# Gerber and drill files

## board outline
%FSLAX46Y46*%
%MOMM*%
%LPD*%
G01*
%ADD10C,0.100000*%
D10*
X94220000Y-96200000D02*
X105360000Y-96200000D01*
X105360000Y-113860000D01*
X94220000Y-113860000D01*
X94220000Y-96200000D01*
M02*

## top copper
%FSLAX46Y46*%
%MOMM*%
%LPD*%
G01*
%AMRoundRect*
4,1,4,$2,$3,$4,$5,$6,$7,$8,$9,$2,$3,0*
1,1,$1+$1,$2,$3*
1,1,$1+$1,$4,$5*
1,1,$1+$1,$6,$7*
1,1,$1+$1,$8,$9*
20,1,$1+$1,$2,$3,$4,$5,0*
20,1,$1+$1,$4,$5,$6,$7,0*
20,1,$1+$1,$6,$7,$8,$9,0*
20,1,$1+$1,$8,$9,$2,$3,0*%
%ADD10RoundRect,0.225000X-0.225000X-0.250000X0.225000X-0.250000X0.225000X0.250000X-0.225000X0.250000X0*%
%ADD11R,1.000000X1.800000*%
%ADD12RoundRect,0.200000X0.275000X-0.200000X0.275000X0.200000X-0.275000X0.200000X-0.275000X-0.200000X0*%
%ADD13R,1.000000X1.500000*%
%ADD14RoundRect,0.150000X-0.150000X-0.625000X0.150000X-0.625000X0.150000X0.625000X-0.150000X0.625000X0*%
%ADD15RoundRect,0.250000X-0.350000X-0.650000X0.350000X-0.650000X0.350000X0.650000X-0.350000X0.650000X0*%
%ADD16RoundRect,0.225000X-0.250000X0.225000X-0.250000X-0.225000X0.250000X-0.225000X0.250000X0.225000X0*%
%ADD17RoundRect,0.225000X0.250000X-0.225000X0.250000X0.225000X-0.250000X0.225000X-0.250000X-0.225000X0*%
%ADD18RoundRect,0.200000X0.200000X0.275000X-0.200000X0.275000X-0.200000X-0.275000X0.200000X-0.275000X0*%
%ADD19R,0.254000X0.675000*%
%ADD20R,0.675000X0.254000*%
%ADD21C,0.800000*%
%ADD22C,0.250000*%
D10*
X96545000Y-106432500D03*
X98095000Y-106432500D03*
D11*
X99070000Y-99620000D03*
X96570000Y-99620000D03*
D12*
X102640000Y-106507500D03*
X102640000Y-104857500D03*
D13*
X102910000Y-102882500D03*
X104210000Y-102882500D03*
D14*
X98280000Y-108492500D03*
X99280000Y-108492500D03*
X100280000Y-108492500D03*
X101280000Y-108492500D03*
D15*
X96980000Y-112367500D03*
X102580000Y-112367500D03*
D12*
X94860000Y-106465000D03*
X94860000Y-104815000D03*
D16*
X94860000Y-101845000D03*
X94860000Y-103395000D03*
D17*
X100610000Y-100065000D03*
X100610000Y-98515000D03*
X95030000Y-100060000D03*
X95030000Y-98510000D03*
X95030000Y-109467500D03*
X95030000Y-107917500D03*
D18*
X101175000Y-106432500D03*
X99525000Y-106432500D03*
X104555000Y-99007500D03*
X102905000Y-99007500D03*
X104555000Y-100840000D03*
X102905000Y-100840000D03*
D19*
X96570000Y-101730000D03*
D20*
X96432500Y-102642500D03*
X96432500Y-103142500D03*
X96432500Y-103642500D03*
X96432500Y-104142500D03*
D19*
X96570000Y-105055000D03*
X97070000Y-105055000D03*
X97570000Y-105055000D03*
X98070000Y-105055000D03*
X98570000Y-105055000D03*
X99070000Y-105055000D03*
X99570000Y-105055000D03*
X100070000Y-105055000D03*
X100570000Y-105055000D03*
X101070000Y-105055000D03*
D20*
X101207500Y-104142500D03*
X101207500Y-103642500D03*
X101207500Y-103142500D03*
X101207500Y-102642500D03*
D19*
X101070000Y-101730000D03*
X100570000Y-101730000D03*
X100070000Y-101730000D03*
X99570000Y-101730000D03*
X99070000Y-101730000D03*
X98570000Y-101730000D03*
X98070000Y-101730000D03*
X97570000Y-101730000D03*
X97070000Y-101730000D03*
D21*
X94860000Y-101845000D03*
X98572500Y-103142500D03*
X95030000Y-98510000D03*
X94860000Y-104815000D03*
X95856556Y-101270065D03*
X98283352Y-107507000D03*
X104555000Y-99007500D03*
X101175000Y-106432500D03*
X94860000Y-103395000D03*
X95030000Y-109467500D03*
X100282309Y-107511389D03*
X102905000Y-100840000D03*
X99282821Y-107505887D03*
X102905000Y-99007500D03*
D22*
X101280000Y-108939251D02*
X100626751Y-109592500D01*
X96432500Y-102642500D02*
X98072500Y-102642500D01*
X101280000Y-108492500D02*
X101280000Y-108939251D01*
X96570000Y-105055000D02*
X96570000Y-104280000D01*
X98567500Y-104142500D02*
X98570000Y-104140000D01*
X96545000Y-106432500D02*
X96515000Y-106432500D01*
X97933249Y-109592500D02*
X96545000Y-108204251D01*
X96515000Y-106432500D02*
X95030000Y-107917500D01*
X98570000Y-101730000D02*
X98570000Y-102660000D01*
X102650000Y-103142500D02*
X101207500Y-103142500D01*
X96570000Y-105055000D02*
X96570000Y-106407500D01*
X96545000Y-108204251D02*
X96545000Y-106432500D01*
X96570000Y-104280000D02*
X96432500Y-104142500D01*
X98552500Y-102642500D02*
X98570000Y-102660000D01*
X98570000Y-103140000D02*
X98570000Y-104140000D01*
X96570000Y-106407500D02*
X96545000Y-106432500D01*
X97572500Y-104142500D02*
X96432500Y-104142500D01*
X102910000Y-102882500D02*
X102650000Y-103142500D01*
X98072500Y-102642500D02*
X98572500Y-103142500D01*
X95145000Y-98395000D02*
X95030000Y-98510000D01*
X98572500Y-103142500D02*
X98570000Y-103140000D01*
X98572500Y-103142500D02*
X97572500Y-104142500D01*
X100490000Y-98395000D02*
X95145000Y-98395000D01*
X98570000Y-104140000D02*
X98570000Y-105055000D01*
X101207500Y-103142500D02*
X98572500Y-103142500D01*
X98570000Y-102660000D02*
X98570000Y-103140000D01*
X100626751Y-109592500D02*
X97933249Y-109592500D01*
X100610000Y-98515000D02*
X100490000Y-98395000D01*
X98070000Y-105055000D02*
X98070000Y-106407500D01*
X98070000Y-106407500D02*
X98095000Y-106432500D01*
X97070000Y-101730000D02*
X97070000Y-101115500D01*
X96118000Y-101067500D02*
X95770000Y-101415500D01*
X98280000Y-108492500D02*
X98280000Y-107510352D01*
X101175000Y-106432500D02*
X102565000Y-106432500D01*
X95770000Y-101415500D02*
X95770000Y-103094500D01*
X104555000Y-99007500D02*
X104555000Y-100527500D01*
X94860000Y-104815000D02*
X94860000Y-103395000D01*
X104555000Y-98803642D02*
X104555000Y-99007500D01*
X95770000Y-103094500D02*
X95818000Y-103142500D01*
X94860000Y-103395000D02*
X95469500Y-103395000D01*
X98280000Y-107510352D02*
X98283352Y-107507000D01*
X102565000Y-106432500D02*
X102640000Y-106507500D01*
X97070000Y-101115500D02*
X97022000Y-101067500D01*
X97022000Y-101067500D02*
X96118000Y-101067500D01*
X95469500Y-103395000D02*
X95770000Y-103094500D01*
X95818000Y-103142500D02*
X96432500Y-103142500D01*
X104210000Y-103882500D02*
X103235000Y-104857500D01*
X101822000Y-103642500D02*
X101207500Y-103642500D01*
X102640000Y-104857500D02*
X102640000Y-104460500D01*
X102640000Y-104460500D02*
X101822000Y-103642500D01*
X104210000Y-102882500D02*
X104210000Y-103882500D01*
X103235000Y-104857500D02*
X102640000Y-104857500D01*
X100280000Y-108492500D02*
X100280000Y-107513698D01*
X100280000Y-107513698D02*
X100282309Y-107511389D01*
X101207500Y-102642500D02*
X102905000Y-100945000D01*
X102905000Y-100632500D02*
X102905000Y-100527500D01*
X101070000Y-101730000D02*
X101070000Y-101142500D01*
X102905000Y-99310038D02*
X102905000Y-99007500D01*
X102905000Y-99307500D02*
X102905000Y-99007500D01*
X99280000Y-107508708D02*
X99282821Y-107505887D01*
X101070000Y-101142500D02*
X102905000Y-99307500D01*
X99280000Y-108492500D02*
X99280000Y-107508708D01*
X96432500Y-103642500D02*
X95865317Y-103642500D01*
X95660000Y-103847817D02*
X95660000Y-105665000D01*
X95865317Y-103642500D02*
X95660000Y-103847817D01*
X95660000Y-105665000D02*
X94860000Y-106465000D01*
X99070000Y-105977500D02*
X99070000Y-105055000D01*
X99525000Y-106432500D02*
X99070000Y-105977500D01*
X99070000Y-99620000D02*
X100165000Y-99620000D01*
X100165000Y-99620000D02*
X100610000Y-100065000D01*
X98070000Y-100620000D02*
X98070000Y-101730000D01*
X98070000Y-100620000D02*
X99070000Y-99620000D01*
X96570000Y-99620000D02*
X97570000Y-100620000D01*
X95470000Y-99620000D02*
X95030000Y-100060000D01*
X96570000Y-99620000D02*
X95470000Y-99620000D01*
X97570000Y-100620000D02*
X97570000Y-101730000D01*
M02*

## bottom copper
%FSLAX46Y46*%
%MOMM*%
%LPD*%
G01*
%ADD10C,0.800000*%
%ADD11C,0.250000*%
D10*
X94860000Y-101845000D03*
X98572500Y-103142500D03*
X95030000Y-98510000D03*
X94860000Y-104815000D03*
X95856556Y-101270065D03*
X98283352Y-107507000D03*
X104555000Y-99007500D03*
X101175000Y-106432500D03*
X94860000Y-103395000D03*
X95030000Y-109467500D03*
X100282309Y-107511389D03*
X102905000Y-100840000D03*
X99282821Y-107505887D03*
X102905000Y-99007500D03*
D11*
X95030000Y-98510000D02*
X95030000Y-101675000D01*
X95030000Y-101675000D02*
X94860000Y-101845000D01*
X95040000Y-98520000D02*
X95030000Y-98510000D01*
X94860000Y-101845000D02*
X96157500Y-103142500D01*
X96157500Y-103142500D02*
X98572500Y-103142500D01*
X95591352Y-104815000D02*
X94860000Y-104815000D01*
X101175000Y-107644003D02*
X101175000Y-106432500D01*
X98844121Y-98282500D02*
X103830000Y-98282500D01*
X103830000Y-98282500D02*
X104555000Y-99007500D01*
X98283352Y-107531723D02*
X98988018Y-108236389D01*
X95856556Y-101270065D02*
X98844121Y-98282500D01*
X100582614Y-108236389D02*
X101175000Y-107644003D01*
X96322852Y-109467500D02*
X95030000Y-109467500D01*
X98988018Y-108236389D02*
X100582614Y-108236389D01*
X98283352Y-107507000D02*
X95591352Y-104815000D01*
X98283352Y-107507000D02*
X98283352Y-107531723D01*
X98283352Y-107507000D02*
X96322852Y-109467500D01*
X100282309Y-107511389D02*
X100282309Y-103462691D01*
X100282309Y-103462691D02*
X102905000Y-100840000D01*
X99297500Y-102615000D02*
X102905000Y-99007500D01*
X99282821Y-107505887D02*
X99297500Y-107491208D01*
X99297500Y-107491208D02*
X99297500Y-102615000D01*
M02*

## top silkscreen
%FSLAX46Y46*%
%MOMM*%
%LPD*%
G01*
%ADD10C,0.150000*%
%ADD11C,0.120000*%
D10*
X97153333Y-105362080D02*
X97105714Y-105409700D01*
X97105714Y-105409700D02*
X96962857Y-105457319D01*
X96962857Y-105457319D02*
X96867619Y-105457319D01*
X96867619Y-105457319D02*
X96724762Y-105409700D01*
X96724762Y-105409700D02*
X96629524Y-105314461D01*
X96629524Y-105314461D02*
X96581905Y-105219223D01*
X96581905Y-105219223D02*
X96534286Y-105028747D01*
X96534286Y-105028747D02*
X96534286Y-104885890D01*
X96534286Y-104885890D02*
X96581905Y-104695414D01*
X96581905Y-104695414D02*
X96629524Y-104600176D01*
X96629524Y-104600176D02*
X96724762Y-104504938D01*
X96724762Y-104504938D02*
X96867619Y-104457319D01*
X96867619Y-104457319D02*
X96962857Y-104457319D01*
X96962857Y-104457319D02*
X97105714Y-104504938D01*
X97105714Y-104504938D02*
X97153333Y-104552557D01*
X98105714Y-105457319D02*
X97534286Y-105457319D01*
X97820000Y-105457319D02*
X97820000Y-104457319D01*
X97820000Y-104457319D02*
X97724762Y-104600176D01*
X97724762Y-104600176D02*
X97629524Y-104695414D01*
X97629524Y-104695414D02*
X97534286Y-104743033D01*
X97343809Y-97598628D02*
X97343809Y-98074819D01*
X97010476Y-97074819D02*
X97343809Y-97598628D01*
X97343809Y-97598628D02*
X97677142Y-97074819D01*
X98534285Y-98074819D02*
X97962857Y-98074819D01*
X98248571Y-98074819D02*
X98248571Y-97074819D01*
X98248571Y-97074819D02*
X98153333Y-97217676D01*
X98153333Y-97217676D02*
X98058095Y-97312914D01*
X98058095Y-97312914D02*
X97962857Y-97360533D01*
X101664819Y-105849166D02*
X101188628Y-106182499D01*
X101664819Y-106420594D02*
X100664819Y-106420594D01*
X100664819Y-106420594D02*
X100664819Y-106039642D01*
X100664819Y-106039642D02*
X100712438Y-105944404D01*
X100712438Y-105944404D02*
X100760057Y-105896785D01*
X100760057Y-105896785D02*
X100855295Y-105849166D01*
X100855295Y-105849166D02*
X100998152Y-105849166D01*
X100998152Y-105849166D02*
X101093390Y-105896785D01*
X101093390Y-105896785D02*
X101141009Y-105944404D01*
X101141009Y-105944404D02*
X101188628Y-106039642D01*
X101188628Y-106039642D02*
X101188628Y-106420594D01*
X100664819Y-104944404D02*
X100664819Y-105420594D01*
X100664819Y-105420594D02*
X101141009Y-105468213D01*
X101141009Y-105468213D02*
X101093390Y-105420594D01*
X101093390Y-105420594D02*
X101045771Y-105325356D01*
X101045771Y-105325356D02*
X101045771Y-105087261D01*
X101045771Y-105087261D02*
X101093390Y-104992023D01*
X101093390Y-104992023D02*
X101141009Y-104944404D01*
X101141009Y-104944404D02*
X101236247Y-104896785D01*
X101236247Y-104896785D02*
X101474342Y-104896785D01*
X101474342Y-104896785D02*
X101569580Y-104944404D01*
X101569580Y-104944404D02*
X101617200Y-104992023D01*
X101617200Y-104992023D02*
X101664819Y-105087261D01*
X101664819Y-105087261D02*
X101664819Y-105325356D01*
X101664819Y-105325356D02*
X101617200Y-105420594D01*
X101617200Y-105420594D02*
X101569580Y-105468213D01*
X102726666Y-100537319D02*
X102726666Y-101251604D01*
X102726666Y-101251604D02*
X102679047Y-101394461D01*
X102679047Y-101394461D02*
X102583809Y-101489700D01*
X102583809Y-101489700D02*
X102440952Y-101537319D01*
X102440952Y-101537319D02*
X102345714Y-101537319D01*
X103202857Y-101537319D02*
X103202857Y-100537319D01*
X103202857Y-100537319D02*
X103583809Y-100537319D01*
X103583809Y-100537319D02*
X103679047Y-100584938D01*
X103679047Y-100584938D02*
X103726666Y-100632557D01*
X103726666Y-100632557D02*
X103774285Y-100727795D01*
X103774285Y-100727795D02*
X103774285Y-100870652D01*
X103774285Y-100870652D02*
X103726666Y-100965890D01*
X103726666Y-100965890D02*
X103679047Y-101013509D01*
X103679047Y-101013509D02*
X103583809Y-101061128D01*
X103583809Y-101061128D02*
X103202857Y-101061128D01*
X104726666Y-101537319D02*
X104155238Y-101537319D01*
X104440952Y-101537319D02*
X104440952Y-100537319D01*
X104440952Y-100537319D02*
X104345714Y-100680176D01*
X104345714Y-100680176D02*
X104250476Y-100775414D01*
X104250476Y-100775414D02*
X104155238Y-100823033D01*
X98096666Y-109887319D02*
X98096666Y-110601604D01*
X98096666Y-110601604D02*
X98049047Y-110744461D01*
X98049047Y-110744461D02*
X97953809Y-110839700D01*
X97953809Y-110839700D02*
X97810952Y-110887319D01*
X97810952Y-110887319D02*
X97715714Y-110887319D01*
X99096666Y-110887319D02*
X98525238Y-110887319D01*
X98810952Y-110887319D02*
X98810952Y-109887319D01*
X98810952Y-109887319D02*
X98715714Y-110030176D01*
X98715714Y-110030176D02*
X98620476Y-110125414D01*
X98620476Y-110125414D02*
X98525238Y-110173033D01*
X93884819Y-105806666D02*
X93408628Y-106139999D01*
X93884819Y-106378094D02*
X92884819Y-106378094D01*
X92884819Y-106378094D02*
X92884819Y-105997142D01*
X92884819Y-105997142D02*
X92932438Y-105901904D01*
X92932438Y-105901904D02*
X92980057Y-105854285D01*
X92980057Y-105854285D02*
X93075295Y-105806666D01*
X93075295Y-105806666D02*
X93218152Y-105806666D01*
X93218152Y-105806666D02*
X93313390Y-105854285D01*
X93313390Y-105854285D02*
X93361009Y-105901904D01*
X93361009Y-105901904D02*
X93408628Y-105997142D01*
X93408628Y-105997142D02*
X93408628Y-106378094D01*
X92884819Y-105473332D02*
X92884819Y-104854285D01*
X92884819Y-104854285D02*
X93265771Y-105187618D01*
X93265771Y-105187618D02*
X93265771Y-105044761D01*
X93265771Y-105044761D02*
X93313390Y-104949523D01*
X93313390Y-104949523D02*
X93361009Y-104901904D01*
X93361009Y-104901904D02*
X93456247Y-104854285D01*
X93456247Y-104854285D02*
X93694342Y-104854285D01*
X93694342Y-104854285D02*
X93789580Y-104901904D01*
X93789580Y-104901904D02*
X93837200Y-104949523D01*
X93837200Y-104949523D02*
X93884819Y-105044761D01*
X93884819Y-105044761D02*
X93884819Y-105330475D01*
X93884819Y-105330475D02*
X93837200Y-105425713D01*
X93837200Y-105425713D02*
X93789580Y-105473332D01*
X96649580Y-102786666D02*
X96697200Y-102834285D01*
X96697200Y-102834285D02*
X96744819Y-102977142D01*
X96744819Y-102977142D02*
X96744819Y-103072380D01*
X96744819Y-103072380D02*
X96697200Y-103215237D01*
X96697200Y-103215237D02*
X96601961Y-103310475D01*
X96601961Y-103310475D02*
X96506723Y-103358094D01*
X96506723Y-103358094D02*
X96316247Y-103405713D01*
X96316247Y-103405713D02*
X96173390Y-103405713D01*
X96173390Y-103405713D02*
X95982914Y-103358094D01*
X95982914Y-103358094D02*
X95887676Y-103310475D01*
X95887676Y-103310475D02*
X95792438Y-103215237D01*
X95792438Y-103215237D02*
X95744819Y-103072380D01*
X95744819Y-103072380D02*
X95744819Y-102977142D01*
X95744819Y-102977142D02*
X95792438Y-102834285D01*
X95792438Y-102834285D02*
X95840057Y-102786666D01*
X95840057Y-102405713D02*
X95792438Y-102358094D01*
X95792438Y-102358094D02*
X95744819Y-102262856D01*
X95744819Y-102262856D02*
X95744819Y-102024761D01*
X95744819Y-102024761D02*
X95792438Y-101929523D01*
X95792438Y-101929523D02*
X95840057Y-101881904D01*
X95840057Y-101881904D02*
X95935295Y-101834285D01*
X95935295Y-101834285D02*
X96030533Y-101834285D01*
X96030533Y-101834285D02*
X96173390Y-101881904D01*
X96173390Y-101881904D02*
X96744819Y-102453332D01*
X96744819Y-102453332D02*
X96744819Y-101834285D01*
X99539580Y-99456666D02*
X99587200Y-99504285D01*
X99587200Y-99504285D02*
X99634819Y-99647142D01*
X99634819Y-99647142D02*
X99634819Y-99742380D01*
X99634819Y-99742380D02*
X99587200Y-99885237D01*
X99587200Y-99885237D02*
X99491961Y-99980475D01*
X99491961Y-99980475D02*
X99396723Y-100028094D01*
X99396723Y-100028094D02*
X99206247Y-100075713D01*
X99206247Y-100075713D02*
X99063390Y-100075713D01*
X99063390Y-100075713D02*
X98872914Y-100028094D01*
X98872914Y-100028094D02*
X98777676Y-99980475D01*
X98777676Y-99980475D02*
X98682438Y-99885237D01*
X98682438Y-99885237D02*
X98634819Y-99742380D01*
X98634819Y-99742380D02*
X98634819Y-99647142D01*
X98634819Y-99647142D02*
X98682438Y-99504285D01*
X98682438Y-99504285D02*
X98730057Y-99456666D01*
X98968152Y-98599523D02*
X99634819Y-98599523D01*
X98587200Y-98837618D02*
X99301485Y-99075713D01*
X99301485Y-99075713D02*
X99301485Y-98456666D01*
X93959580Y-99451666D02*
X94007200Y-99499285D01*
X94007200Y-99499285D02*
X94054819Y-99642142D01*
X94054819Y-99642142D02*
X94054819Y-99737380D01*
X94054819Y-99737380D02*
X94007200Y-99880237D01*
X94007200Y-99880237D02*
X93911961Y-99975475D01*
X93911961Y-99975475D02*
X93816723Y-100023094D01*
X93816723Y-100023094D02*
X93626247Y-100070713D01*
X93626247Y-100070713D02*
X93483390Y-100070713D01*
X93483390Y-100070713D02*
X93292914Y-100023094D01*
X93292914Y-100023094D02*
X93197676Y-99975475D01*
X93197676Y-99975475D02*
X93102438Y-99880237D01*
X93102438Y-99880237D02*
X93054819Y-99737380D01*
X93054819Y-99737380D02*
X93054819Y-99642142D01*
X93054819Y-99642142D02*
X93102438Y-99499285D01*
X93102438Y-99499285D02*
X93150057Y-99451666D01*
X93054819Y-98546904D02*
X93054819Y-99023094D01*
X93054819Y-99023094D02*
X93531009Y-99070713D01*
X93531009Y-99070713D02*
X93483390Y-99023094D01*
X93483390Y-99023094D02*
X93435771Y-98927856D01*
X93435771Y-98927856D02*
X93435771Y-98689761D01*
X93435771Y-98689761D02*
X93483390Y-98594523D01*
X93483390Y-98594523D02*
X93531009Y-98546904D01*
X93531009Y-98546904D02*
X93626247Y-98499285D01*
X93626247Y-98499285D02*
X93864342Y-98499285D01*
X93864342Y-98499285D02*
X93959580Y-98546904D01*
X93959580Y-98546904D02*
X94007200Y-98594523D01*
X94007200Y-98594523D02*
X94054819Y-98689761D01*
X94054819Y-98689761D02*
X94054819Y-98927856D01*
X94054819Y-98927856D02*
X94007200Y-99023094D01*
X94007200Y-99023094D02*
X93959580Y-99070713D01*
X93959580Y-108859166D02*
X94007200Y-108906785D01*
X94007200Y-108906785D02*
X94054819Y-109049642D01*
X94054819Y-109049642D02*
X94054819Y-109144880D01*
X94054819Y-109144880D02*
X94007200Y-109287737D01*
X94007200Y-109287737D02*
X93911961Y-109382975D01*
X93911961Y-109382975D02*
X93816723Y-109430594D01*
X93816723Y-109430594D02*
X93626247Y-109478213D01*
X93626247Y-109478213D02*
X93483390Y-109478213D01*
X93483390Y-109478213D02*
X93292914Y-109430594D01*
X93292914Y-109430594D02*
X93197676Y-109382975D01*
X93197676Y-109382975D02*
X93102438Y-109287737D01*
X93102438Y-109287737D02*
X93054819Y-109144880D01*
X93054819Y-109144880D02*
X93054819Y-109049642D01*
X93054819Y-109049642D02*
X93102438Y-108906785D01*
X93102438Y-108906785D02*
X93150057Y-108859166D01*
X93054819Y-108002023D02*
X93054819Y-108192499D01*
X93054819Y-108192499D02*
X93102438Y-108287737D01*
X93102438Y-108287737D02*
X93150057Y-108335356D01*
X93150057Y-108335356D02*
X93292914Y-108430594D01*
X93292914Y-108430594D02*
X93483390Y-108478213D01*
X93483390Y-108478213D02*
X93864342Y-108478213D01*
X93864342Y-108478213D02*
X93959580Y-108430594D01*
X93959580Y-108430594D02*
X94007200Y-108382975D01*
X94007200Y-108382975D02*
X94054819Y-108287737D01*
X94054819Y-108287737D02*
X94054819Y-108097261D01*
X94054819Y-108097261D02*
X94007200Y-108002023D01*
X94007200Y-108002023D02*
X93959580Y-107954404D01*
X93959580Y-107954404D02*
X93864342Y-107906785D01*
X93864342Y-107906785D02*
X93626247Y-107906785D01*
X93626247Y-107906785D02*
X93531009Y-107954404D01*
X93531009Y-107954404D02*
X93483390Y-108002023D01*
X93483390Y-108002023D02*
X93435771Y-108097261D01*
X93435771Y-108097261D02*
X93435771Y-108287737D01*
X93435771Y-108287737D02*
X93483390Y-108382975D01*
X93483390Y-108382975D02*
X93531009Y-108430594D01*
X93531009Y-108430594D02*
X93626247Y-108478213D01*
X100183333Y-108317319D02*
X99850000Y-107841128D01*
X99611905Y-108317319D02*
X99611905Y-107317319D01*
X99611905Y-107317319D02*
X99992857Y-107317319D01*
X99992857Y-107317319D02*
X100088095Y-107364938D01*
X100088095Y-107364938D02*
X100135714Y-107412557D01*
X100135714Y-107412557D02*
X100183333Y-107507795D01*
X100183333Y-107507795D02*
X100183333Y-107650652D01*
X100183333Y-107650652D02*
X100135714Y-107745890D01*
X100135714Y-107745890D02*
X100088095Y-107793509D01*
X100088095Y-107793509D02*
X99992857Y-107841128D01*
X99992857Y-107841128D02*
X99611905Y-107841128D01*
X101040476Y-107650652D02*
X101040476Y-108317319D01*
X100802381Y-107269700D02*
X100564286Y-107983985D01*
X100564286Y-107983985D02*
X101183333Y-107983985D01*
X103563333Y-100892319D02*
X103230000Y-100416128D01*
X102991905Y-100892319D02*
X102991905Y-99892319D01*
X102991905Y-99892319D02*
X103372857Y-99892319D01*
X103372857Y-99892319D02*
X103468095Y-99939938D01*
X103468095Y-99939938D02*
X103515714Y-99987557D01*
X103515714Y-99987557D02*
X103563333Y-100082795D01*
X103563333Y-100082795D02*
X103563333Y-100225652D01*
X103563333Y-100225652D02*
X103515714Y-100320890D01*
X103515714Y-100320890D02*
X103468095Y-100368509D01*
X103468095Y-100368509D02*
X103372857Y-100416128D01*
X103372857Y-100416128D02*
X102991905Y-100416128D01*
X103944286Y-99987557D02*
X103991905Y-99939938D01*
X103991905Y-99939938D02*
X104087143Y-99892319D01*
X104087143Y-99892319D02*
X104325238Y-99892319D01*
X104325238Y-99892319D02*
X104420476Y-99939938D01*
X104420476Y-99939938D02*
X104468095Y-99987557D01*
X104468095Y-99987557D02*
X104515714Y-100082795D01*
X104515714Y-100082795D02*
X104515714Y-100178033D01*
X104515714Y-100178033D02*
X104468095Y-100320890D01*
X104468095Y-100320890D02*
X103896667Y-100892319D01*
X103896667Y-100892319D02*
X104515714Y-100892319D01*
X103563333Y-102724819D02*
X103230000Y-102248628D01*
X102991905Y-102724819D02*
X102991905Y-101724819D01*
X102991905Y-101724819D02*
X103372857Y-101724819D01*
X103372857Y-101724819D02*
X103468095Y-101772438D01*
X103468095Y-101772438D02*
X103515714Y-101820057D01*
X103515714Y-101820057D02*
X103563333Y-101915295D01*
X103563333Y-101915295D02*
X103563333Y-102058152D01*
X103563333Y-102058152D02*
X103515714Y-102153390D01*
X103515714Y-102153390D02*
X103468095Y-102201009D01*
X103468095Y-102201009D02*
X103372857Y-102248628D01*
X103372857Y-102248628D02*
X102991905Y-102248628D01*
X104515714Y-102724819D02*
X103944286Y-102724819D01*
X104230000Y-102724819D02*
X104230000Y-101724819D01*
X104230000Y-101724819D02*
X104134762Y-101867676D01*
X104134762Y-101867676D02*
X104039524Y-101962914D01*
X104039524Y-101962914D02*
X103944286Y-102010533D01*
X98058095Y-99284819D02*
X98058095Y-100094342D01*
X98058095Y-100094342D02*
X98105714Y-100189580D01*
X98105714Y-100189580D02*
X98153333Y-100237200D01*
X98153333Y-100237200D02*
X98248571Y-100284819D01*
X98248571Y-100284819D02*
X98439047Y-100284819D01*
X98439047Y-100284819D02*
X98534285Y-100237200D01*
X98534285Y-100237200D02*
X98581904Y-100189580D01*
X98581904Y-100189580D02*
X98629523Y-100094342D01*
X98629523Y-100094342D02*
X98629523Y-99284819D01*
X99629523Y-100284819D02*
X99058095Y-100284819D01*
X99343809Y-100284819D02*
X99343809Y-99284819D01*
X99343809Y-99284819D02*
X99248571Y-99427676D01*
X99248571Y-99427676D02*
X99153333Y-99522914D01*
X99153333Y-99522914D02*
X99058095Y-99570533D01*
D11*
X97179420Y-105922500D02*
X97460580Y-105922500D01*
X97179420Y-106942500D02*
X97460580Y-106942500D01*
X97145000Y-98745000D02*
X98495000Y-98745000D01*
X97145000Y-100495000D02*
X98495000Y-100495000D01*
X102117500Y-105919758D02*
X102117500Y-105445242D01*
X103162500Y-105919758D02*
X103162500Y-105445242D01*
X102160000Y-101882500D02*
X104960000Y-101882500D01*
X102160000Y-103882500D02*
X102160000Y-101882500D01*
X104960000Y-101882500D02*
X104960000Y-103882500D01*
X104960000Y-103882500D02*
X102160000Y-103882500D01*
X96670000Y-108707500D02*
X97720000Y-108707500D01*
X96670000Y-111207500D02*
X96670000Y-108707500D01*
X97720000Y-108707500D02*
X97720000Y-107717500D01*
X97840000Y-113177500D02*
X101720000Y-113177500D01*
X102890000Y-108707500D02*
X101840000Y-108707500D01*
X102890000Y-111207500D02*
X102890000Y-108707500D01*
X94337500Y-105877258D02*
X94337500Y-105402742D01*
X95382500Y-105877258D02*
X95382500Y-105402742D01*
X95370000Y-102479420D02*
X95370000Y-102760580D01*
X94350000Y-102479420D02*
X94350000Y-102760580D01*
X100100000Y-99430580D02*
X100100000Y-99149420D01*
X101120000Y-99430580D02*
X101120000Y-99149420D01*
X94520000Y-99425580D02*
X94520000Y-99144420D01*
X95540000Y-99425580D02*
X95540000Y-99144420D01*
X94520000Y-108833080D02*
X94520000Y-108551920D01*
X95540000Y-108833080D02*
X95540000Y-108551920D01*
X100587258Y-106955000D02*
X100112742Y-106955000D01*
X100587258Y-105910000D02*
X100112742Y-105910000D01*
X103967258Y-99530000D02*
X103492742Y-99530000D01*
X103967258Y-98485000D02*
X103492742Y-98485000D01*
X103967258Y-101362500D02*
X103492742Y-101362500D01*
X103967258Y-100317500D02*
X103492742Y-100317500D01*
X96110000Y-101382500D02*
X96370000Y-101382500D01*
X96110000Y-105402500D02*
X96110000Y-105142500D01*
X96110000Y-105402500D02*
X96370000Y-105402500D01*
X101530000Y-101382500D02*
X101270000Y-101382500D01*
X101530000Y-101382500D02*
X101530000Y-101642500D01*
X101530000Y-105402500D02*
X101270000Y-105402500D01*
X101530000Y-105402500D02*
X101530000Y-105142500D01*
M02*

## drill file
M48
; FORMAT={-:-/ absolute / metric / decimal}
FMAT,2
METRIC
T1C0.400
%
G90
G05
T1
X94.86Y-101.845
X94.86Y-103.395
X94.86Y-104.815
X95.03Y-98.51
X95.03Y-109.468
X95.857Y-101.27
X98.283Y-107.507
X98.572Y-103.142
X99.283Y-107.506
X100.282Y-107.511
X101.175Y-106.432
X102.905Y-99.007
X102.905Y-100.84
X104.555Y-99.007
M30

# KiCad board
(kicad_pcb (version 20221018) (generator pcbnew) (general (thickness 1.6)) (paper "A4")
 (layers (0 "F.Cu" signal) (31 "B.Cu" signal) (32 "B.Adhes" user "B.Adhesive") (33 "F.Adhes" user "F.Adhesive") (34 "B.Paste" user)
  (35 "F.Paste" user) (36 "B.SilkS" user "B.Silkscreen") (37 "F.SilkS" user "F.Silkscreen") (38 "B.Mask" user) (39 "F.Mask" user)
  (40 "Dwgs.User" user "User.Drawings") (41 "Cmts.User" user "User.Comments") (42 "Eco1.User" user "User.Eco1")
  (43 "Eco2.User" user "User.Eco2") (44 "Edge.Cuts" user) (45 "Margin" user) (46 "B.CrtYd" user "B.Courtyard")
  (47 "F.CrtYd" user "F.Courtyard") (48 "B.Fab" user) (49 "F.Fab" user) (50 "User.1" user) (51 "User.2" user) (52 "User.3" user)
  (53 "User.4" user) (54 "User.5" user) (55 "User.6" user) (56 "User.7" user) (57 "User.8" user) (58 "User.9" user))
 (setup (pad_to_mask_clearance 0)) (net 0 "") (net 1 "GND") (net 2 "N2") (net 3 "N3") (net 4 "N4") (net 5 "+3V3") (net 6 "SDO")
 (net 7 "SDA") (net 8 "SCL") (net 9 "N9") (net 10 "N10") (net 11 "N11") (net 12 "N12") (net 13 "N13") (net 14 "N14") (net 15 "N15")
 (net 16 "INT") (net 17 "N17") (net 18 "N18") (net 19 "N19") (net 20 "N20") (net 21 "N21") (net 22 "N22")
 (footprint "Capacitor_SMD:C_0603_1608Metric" (layer "F.Cu") (at 97.32 106.4325)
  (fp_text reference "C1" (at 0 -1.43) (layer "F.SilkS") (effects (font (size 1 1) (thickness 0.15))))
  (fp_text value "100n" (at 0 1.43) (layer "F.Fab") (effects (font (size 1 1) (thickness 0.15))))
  (fp_line (start -0.14058 -0.51) (end 0.14058 -0.51) (stroke (width 0.12) (type solid)) (layer "F.SilkS"))
  (fp_line (start -0.14058 0.51) (end 0.14058 0.51) (stroke (width 0.12) (type solid)) (layer "F.SilkS"))
  (pad "1" smd roundrect (at -0.775 0) (size 0.9 0.95) (layers "F.Cu" "F.Paste" "F.Mask") (roundrect_rratio 0.25) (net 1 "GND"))
  (pad "2" smd roundrect (at 0.775 0) (size 0.9 0.95) (layers "F.Cu" "F.Paste" "F.Mask") (roundrect_rratio 0.25) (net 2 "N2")))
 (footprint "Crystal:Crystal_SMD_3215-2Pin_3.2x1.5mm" (layer "F.Cu") (at 97.82 99.62)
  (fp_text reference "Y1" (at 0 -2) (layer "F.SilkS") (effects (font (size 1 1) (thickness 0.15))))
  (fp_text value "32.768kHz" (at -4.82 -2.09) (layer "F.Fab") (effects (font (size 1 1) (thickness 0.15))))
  (fp_line (start -0.675 -0.875) (end 0.675 -0.875) (stroke (width 0.12) (type solid)) (layer "F.SilkS"))
  (fp_line (start -0.675 0.875) (end 0.675 0.875) (stroke (width 0.12) (type solid)) (layer "F.SilkS"))
  (pad "1" smd rect (at 1.25 0) (size 1 1.8) (layers "F.Cu" "F.Paste" "F.Mask") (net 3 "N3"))
  (pad "2" smd rect (at -1.25 0) (size 1 1.8) (layers "F.Cu" "F.Paste" "F.Mask") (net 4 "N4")))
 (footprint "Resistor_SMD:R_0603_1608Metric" (layer "F.Cu") (at 102.64 105.6825 90)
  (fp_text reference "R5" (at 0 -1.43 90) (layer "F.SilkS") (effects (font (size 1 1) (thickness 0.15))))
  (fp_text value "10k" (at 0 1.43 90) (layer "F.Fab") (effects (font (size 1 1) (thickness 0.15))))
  (fp_line (start -0.237258 -0.5225) (end 0.237258 -0.5225) (stroke (width 0.12) (type solid)) (layer "F.SilkS"))
  (fp_line (start -0.237258 0.5225) (end 0.237258 0.5225) (stroke (width 0.12) (type solid)) (layer "F.SilkS"))
  (pad "1" smd roundrect (at -0.825 0 90) (size 0.8 0.95) (layers "F.Cu" "F.Paste" "F.Mask") (roundrect_rratio 0.25) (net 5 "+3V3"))
  (pad "2" smd roundrect (at 0.825 0 90) (size 0.8 0.95) (layers "F.Cu" "F.Paste" "F.Mask") (roundrect_rratio 0.25) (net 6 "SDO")))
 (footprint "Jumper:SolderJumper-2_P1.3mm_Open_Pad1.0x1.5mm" (layer "F.Cu") (at 103.56 102.8825)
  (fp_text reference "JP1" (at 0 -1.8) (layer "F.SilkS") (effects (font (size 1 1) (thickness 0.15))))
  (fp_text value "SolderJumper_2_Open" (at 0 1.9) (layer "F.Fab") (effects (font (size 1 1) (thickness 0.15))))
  (fp_line (start -1.4 -1) (end 1.4 -1) (stroke (width 0.12) (type solid)) (layer "F.SilkS"))
  (fp_line (start -1.4 1) (end -1.4 -1) (stroke (width 0.12) (type solid)) (layer "F.SilkS"))
  (fp_line (start 1.4 -1) (end 1.4 1) (stroke (width 0.12) (type solid)) (layer "F.SilkS"))
  (fp_line (start 1.4 1) (end -1.4 1) (stroke (width 0.12) (type solid)) (layer "F.SilkS"))
  (pad "1" smd rect (at -0.65 0) (size 1 1.5) (layers "F.Cu" "F.Mask") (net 1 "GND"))
  (pad "2" smd rect (at 0.65 0) (size 1 1.5) (layers "F.Cu" "F.Mask") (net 6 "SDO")))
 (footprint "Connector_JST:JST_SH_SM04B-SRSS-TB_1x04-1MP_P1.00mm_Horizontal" (layer "F.Cu") (at 99.78 110.4925)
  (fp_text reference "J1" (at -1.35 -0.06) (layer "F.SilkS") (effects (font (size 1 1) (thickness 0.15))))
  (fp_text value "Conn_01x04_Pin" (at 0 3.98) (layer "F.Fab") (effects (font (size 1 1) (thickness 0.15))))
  (fp_line (start -3.11 -1.785) (end -2.06 -1.785) (stroke (width 0.12) (type solid)) (layer "F.SilkS"))
  (fp_line (start -3.11 0.715) (end -3.11 -1.785) (stroke (width 0.12) (type solid)) (layer "F.SilkS"))
  (fp_line (start -2.06 -1.785) (end -2.06 -2.775) (stroke (width 0.12) (type solid)) (layer "F.SilkS"))
  (fp_line (start -1.94 2.685) (end 1.94 2.685) (stroke (width 0.12) (type solid)) (layer "F.SilkS"))
  (fp_line (start 3.11 -1.785) (end 2.06 -1.785) (stroke (width 0.12) (type solid)) (layer "F.SilkS"))
  (fp_line (start 3.11 0.715) (end 3.11 -1.785) (stroke (width 0.12) (type solid)) (layer "F.SilkS"))
  (pad "1" smd roundrect (at -1.5 -2) (size 0.6 1.55) (layers "F.Cu" "F.Paste" "F.Mask") (roundrect_rratio 0.25) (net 5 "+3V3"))
  (pad "2" smd roundrect (at -0.5 -2) (size 0.6 1.55) (layers "F.Cu" "F.Paste" "F.Mask") (roundrect_rratio 0.25) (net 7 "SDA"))
  (pad "3" smd roundrect (at 0.5 -2) (size 0.6 1.55) (layers "F.Cu" "F.Paste" "F.Mask") (roundrect_rratio 0.25) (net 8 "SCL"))
  (pad "4" smd roundrect (at 1.5 -2) (size 0.6 1.55) (layers "F.Cu" "F.Paste" "F.Mask") (roundrect_rratio 0.25) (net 1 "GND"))
  (pad "MP" smd roundrect (at -2.8 1.875) (size 1.2 1.8) (layers "F.Cu" "F.Paste" "F.Mask") (roundrect_rratio 0.208333))
  (pad "MP" smd roundrect (at 2.8 1.875) (size 1.2 1.8) (layers "F.Cu" "F.Paste" "F.Mask") (roundrect_rratio 0.208333)))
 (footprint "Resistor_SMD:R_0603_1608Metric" (layer "F.Cu") (at 94.86 105.64 90)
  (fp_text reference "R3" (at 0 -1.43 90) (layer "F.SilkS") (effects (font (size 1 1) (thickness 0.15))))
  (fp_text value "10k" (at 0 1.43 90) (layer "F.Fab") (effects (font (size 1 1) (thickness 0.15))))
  (fp_line (start -0.237258 -0.5225) (end 0.237258 -0.5225) (stroke (width 0.12) (type solid)) (layer "F.SilkS"))
  (fp_line (start -0.237258 0.5225) (end 0.237258 0.5225) (stroke (width 0.12) (type solid)) (layer "F.SilkS"))
  (pad "1" smd roundrect (at -0.825 0 90) (size 0.8 0.95) (layers "F.Cu" "F.Paste" "F.Mask") (roundrect_rratio 0.25) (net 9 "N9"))
  (pad "2" smd roundrect (at 0.825 0 90) (size 0.8 0.95) (layers "F.Cu" "F.Paste" "F.Mask") (roundrect_rratio 0.25) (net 5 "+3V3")))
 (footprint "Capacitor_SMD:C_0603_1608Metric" (layer "F.Cu") (at 94.86 102.62 -90)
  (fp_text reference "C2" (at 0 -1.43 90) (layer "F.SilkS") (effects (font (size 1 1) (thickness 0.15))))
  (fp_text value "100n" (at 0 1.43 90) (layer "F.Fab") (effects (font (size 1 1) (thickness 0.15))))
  (fp_line (start -0.14058 -0.51) (end 0.14058 -0.51) (stroke (width 0.12) (type solid)) (layer "F.SilkS"))
  (fp_line (start -0.14058 0.51) (end 0.14058 0.51) (stroke (width 0.12) (type solid)) (layer "F.SilkS"))
  (pad "1" smd roundrect (at -0.775 0 270) (size 0.9 0.95) (layers "F.Cu" "F.Paste" "F.Mask") (roundrect_rratio 0.25) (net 1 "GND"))
  (pad "2" smd roundrect (at 0.775 0 270) (size 0.9 0.95) (layers "F.Cu" "F.Paste" "F.Mask") (roundrect_rratio 0.25) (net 5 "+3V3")))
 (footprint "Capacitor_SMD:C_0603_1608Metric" (layer "F.Cu") (at 100.61 99.29 90)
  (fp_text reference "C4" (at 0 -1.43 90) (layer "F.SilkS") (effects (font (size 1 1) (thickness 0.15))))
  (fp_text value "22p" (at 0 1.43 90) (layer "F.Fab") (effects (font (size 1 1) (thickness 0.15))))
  (fp_line (start -0.14058 -0.51) (end 0.14058 -0.51) (stroke (width 0.12) (type solid)) (layer "F.SilkS"))
  (fp_line (start -0.14058 0.51) (end 0.14058 0.51) (stroke (width 0.12) (type solid)) (layer "F.SilkS"))
  (pad "1" smd roundrect (at -0.775 0 90) (size 0.9 0.95) (layers "F.Cu" "F.Paste" "F.Mask") (roundrect_rratio 0.25) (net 3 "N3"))
  (pad "2" smd roundrect (at 0.775 0 90) (size 0.9 0.95) (layers "F.Cu" "F.Paste" "F.Mask") (roundrect_rratio 0.25) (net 1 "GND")))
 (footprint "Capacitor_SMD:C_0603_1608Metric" (layer "F.Cu") (at 95.03 99.285 90)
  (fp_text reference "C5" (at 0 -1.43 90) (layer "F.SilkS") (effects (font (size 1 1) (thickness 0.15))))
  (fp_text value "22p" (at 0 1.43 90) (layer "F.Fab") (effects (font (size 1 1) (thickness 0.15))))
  (fp_line (start -0.14058 -0.51) (end 0.14058 -0.51) (stroke (width 0.12) (type solid)) (layer "F.SilkS"))
  (fp_line (start -0.14058 0.51) (end 0.14058 0.51) (stroke (width 0.12) (type solid)) (layer "F.SilkS"))
  (pad "1" smd roundrect (at -0.775 0 90) (size 0.9 0.95) (layers "F.Cu" "F.Paste" "F.Mask") (roundrect_rratio 0.25) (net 4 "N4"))
  (pad "2" smd roundrect (at 0.775 0 90) (size 0.9 0.95) (layers "F.Cu" "F.Paste" "F.Mask") (roundrect_rratio 0.25) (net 1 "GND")))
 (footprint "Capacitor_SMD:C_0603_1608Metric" (layer "F.Cu") (at 95.03 108.6925 90)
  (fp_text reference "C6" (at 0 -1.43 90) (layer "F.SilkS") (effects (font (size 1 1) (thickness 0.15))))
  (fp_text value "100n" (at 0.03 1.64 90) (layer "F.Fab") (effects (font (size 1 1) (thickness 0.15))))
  (fp_line (start -0.14058 -0.51) (end 0.14058 -0.51) (stroke (width 0.12) (type solid)) (layer "F.SilkS"))
  (fp_line (start -0.14058 0.51) (end 0.14058 0.51) (stroke (width 0.12) (type solid)) (layer "F.SilkS"))
  (pad "1" smd roundrect (at -0.775 0 90) (size 0.9 0.95) (layers "F.Cu" "F.Paste" "F.Mask") (roundrect_rratio 0.25) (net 5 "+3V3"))
  (pad "2" smd roundrect (at 0.775 0 90) (size 0.9 0.95) (layers "F.Cu" "F.Paste" "F.Mask") (roundrect_rratio 0.25) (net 1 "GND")))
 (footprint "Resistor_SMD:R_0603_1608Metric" (layer "F.Cu") (at 100.35 106.4325 180)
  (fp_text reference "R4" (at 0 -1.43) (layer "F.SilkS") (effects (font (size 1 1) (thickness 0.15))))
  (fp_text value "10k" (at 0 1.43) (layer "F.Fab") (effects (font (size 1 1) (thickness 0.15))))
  (fp_line (start -0.237258 -0.5225) (end 0.237258 -0.5225) (stroke (width 0.12) (type solid)) (layer "F.SilkS"))
  (fp_line (start -0.237258 0.5225) (end 0.237258 0.5225) (stroke (width 0.12) (type solid)) (layer "F.SilkS"))
  (pad "1" smd roundrect (at -0.825 0 180) (size 0.8 0.95) (layers "F.Cu" "F.Paste" "F.Mask") (roundrect_rratio 0.25) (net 5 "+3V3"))
  (pad "2" smd roundrect (at 0.825 0 180) (size 0.8 0.95) (layers "F.Cu" "F.Paste" "F.Mask") (roundrect_rratio 0.25) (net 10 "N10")))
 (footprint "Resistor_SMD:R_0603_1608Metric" (layer "F.Cu") (at 103.73 99.0075 180)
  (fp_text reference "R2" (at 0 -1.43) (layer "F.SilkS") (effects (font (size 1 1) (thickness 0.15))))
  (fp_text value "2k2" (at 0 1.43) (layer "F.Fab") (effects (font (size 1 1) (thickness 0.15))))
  (fp_line (start -0.237258 -0.5225) (end 0.237258 -0.5225) (stroke (width 0.12) (type solid)) (layer "F.SilkS"))
  (fp_line (start -0.237258 0.5225) (end 0.237258 0.5225) (stroke (width 0.12) (type solid)) (layer "F.SilkS"))
  (pad "1" smd roundrect (at -0.825 0 180) (size 0.8 0.95) (layers "F.Cu" "F.Paste" "F.Mask") (roundrect_rratio 0.25) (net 5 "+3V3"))
  (pad "2" smd roundrect (at 0.825 0 180) (size 0.8 0.95) (layers "F.Cu" "F.Paste" "F.Mask") (roundrect_rratio 0.25) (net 7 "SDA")))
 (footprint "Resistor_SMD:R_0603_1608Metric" (layer "F.Cu") (at 103.73 100.84 180)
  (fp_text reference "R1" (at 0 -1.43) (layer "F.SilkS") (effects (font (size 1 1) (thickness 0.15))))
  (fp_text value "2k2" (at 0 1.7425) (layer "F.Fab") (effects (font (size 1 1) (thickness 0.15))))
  (fp_line (start -0.237258 -0.5225) (end 0.237258 -0.5225) (stroke (width 0.12) (type solid)) (layer "F.SilkS"))
  (fp_line (start -0.237258 0.5225) (end 0.237258 0.5225) (stroke (width 0.12) (type solid)) (layer "F.SilkS"))
  (pad "1" smd roundrect (at -0.825 0 180) (size 0.8 0.95) (layers "F.Cu" "F.Paste" "F.Mask") (roundrect_rratio 0.25) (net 5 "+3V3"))
  (pad "2" smd roundrect (at 0.825 0 180) (size 0.8 0.95) (layers "F.Cu" "F.Paste" "F.Mask") (roundrect_rratio 0.25) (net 8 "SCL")))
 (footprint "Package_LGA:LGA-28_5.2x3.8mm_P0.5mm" (layer "F.Cu") (at 98.82 103.3925)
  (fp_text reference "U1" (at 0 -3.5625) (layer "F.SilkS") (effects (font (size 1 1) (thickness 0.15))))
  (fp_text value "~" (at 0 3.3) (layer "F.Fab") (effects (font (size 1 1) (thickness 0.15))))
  (fp_line (start -2.71 -2.01) (end -2.45 -2.01) (stroke (width 0.12) (type solid)) (layer "F.SilkS"))
  (fp_line (start -2.71 2.01) (end -2.71 1.75) (stroke (width 0.12) (type solid)) (layer "F.SilkS"))
  (fp_line (start -2.71 2.01) (end -2.45 2.01) (stroke (width 0.12) (type solid)) (layer "F.SilkS"))
  (fp_line (start 2.71 -2.01) (end 2.45 -2.01) (stroke (width 0.12) (type solid)) (layer "F.SilkS"))
  (fp_line (start 2.71 -2.01) (end 2.71 -1.75) (stroke (width 0.12) (type solid)) (layer "F.SilkS"))
  (fp_line (start 2.71 2.01) (end 2.45 2.01) (stroke (width 0.12) (type solid)) (layer "F.SilkS"))
  (fp_line (start 2.71 2.01) (end 2.71 1.75) (stroke (width 0.12) (type solid)) (layer "F.SilkS"))
  (pad "1" smd rect (at -2.25 -1.6625) (size 0.254 0.675) (layers "F.Cu" "F.Paste" "F.Mask") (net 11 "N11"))
  (pad "2" smd rect (at -2.3875 -0.75 90) (size 0.254 0.675) (layers "F.Cu" "F.Paste" "F.Mask") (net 1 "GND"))
  (pad "3" smd rect (at -2.3875 -0.25 90) (size 0.254 0.675) (layers "F.Cu" "F.Paste" "F.Mask") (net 5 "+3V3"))
  (pad "4" smd rect (at -2.3875 0.25 90) (size 0.254 0.675) (layers "F.Cu" "F.Paste" "F.Mask") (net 9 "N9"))
  (pad "5" smd rect (at -2.3875 0.75 90) (size 0.254 0.675) (layers "F.Cu" "F.Paste" "F.Mask") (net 1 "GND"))
  (pad "6" smd rect (at -2.25 1.6625) (size 0.254 0.675) (layers "F.Cu" "F.Paste" "F.Mask") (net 1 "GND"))
  (pad "7" smd rect (at -1.75 1.6625) (size 0.254 0.675) (layers "F.Cu" "F.Paste" "F.Mask") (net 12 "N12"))
  (pad "8" smd rect (at -1.25 1.6625) (size 0.254 0.675) (layers "F.Cu" "F.Paste" "F.Mask") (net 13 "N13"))
  (pad "9" smd rect (at -0.75 1.6625) (size 0.254 0.675) (layers "F.Cu" "F.Paste" "F.Mask") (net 2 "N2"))
  (pad "10" smd rect (at -0.25 1.6625) (size 0.254 0.675) (layers "F.Cu" "F.Paste" "F.Mask") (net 1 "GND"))
  (pad "11" smd rect (at 0.25 1.6625) (size 0.254 0.675) (layers "F.Cu" "F.Paste" "F.Mask") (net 10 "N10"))
  (pad "12" smd rect (at 0.75 1.6625) (size 0.254 0.675) (layers "F.Cu" "F.Paste" "F.Mask") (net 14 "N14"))
  (pad "13" smd rect (at 1.25 1.6625) (size 0.254 0.675) (layers "F.Cu" "F.Paste" "F.Mask") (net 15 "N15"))
  (pad "14" smd rect (at 1.75 1.6625) (size 0.254 0.675) (layers "F.Cu" "F.Paste" "F.Mask") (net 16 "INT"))
  (pad "15" smd rect (at 2.25 1.6625) (size 0.254 0.675) (layers "F.Cu" "F.Paste" "F.Mask") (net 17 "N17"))
  (pad "16" smd rect (at 2.3875 0.75 90) (size 0.254 0.675) (layers "F.Cu" "F.Paste" "F.Mask") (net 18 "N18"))
  (pad "17" smd rect (at 2.3875 0.25 90) (size 0.254 0.675) (layers "F.Cu" "F.Paste" "F.Mask") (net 6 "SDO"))
  (pad "18" smd rect (at 2.3875 -0.25 90) (size 0.254 0.675) (layers "F.Cu" "F.Paste" "F.Mask") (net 1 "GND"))
  (pad "19" smd rect (at 2.3875 -0.75 90) (size 0.254 0.675) (layers "F.Cu" "F.Paste" "F.Mask") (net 8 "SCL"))
  (pad "20" smd rect (at 2.25 -1.6625) (size 0.254 0.675) (layers "F.Cu" "F.Paste" "F.Mask") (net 7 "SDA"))
  (pad "21" smd rect (at 1.75 -1.6625) (size 0.254 0.675) (layers "F.Cu" "F.Paste" "F.Mask") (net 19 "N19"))
  (pad "22" smd rect (at 1.25 -1.6625) (size 0.254 0.675) (layers "F.Cu" "F.Paste" "F.Mask") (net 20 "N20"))
  (pad "23" smd rect (at 0.75 -1.6625) (size 0.254 0.675) (layers "F.Cu" "F.Paste" "F.Mask") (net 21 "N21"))
  (pad "24" smd rect (at 0.25 -1.6625) (size 0.254 0.675) (layers "F.Cu" "F.Paste" "F.Mask") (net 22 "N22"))
  (pad "25" smd rect (at -0.25 -1.6625) (size 0.254 0.675) (layers "F.Cu" "F.Paste" "F.Mask") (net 1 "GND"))
  (pad "26" smd rect (at -0.75 -1.6625) (size 0.254 0.675) (layers "F.Cu" "F.Paste" "F.Mask") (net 3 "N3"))
  (pad "27" smd rect (at -1.25 -1.6625) (size 0.254 0.675) (layers "F.Cu" "F.Paste" "F.Mask") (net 4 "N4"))
  (pad "28" smd rect (at -1.75 -1.6625) (size 0.254 0.675) (layers "F.Cu" "F.Paste" "F.Mask") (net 5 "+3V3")))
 (gr_rect (start 94.22 96.2) (end 105.36 113.86) (stroke (width 0.1) (type default)) (fill none) (layer "Edge.Cuts"))
 (segment (start 101.28 108.939251) (end 100.626751 109.5925) (width 0.25) (layer "F.Cu") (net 1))
 (segment (start 96.4325 102.6425) (end 98.0725 102.6425) (width 0.25) (layer "F.Cu") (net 1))
 (segment (start 101.28 108.4925) (end 101.28 108.939251) (width 0.25) (layer "F.Cu") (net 1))
 (segment (start 96.57 105.055) (end 96.57 104.28) (width 0.25) (layer "F.Cu") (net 1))
 (segment (start 98.5675 104.1425) (end 98.57 104.14) (width 0.25) (layer "F.Cu") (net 1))
 (segment (start 96.545 106.4325) (end 96.515 106.4325) (width 0.25) (layer "F.Cu") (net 1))
 (segment (start 97.933249 109.5925) (end 96.545 108.204251) (width 0.25) (layer "F.Cu") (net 1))
 (segment (start 96.515 106.4325) (end 95.03 107.9175) (width 0.25) (layer "F.Cu") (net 1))
 (segment (start 98.57 101.73) (end 98.57 102.66) (width 0.25) (layer "F.Cu") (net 1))
 (segment (start 102.65 103.1425) (end 101.2075 103.1425) (width 0.25) (layer "F.Cu") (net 1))
 (segment (start 96.57 105.055) (end 96.57 106.4075) (width 0.25) (layer "F.Cu") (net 1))
 (segment (start 96.545 108.204251) (end 96.545 106.4325) (width 0.25) (layer "F.Cu") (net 1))
 (segment (start 96.57 104.28) (end 96.4325 104.1425) (width 0.25) (layer "F.Cu") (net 1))
 (segment (start 98.5525 102.6425) (end 98.57 102.66) (width 0.25) (layer "F.Cu") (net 1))
 (segment (start 98.57 103.14) (end 98.57 104.14) (width 0.25) (layer "F.Cu") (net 1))
 (segment (start 96.57 106.4075) (end 96.545 106.4325) (width 0.25) (layer "F.Cu") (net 1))
 (segment (start 97.5725 104.1425) (end 96.4325 104.1425) (width 0.25) (layer "F.Cu") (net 1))
 (segment (start 102.91 102.8825) (end 102.65 103.1425) (width 0.25) (layer "F.Cu") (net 1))
 (segment (start 98.0725 102.6425) (end 98.5725 103.1425) (width 0.25) (layer "F.Cu") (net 1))
 (segment (start 95.145 98.395) (end 95.03 98.51) (width 0.25) (layer "F.Cu") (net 1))
 (segment (start 98.5725 103.1425) (end 98.57 103.14) (width 0.25) (layer "F.Cu") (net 1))
 (segment (start 98.5725 103.1425) (end 97.5725 104.1425) (width 0.25) (layer "F.Cu") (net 1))
 (segment (start 100.49 98.395) (end 95.145 98.395) (width 0.25) (layer "F.Cu") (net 1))
 (segment (start 98.57 104.14) (end 98.57 105.055) (width 0.25) (layer "F.Cu") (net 1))
 (segment (start 101.2075 103.1425) (end 98.5725 103.1425) (width 0.25) (layer "F.Cu") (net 1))
 (segment (start 98.57 102.66) (end 98.57 103.14) (width 0.25) (layer "F.Cu") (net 1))
 (segment (start 100.626751 109.5925) (end 97.933249 109.5925) (width 0.25) (layer "F.Cu") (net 1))
 (segment (start 100.61 98.515) (end 100.49 98.395) (width 0.25) (layer "F.Cu") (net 1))
 (via (at 94.86 101.845) (size 0.8) (drill 0.4) (layers "F.Cu" "B.Cu") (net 1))
 (via (at 98.5725 103.1425) (size 0.8) (drill 0.4) (layers "F.Cu" "B.Cu") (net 1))
 (via (at 95.03 98.51) (size 0.8) (drill 0.4) (layers "F.Cu" "B.Cu") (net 1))
 (segment (start 95.03 98.51) (end 95.03 101.675) (width 0.25) (layer "B.Cu") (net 1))
 (segment (start 95.03 101.675) (end 94.86 101.845) (width 0.25) (layer "B.Cu") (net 1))
 (segment (start 95.04 98.52) (end 95.03 98.51) (width 0.25) (layer "B.Cu") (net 1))
 (segment (start 94.86 101.845) (end 96.1575 103.1425) (width 0.25) (layer "B.Cu") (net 1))
 (segment (start 96.1575 103.1425) (end 98.5725 103.1425) (width 0.25) (layer "B.Cu") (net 1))
 (segment (start 98.07 105.055) (end 98.07 106.4075) (width 0.25) (layer "F.Cu") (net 2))
 (segment (start 98.07 106.4075) (end 98.095 106.4325) (width 0.25) (layer "F.Cu") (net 2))
 (segment (start 97.07 101.73) (end 97.07 101.1155) (width 0.25) (layer "F.Cu") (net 5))
 (segment (start 96.118 101.0675) (end 95.77 101.4155) (width 0.25) (layer "F.Cu") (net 5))
 (segment (start 98.28 108.4925) (end 98.28 107.510352) (width 0.25) (layer "F.Cu") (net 5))
 (segment (start 101.175 106.4325) (end 102.565 106.4325) (width 0.25) (layer "F.Cu") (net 5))
 (segment (start 95.77 101.4155) (end 95.77 103.0945) (width 0.25) (layer "F.Cu") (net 5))
 (segment (start 104.555 99.0075) (end 104.555 100.5275) (width 0.25) (layer "F.Cu") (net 5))
 (segment (start 94.86 104.815) (end 94.86 103.395) (width 0.25) (layer "F.Cu") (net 5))
 (segment (start 104.555 98.803642) (end 104.555 99.0075) (width 0.25) (layer "F.Cu") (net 5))
 (segment (start 95.77 103.0945) (end 95.818 103.1425) (width 0.25) (layer "F.Cu") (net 5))
 (segment (start 94.86 103.395) (end 95.4695 103.395) (width 0.25) (layer "F.Cu") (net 5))
 (segment (start 98.28 107.510352) (end 98.283352 107.507) (width 0.25) (layer "F.Cu") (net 5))
 (segment (start 102.565 106.4325) (end 102.64 106.5075) (width 0.25) (layer "F.Cu") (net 5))
 (segment (start 97.07 101.1155) (end 97.022 101.0675) (width 0.25) (layer "F.Cu") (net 5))
 (segment (start 97.022 101.0675) (end 96.118 101.0675) (width 0.25) (layer "F.Cu") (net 5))
 (segment (start 95.4695 103.395) (end 95.77 103.0945) (width 0.25) (layer "F.Cu") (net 5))
 (segment (start 95.818 103.1425) (end 96.4325 103.1425) (width 0.25) (layer "F.Cu") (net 5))
 (via (at 94.86 104.815) (size 0.8) (drill 0.4) (layers "F.Cu" "B.Cu") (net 5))
 (via (at 95.856556 101.270065) (size 0.8) (drill 0.4) (layers "F.Cu" "B.Cu") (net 5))
 (via (at 98.283352 107.507) (size 0.8) (drill 0.4) (layers "F.Cu" "B.Cu") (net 5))
 (via (at 104.555 99.0075) (size 0.8) (drill 0.4) (layers "F.Cu" "B.Cu") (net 5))
 (via (at 101.175 106.4325) (size 0.8) (drill 0.4) (layers "F.Cu" "B.Cu") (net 5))
 (via (at 94.86 103.395) (size 0.8) (drill 0.4) (layers "F.Cu" "B.Cu") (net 5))
 (via (at 95.03 109.4675) (size 0.8) (drill 0.4) (layers "F.Cu" "B.Cu") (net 5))
 (segment (start 95.591352 104.815) (end 94.86 104.815) (width 0.25) (layer "B.Cu") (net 5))
 (segment (start 101.175 107.644003) (end 101.175 106.4325) (width 0.25) (layer "B.Cu") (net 5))
 (segment (start 98.844121 98.2825) (end 103.83 98.2825) (width 0.25) (layer "B.Cu") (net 5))
 (segment (start 103.83 98.2825) (end 104.555 99.0075) (width 0.25) (layer "B.Cu") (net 5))
 (segment (start 98.283352 107.531723) (end 98.988018 108.236389) (width 0.25) (layer "B.Cu") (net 5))
 (segment (start 95.856556 101.270065) (end 98.844121 98.2825) (width 0.25) (layer "B.Cu") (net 5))
 (segment (start 100.582614 108.236389) (end 101.175 107.644003) (width 0.25) (layer "B.Cu") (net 5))
 (segment (start 96.322852 109.4675) (end 95.03 109.4675) (width 0.25) (layer "B.Cu") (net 5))
 (segment (start 98.988018 108.236389) (end 100.582614 108.236389) (width 0.25) (layer "B.Cu") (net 5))
 (segment (start 98.283352 107.507) (end 95.591352 104.815) (width 0.25) (layer "B.Cu") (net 5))
 (segment (start 98.283352 107.507) (end 98.283352 107.531723) (width 0.25) (layer "B.Cu") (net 5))
 (segment (start 98.283352 107.507) (end 96.322852 109.4675) (width 0.25) (layer "B.Cu") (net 5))
 (segment (start 104.21 103.8825) (end 103.235 104.8575) (width 0.25) (layer "F.Cu") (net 6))
 (segment (start 101.822 103.6425) (end 101.2075 103.6425) (width 0.25) (layer "F.Cu") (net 6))
 (segment (start 102.64 104.8575) (end 102.64 104.4605) (width 0.25) (layer "F.Cu") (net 6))
 (segment (start 102.64 104.4605) (end 101.822 103.6425) (width 0.25) (layer "F.Cu") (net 6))
 (segment (start 104.21 102.8825) (end 104.21 103.8825) (width 0.25) (layer "F.Cu") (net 6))
 (segment (start 103.235 104.8575) (end 102.64 104.8575) (width 0.25) (layer "F.Cu") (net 6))
 (segment (start 100.28 108.4925) (end 100.28 107.513698) (width 0.25) (layer "F.Cu") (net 8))
 (segment (start 100.28 107.513698) (end 100.282309 107.511389) (width 0.25) (layer "F.Cu") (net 8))
 (segment (start 101.2075 102.6425) (end 102.905 100.945) (width 0.25) (layer "F.Cu") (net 8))
 (segment (start 102.905 100.6325) (end 102.905 100.5275) (width 0.25) (layer "F.Cu") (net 8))
 (via (at 100.282309 107.511389) (size 0.8) (drill 0.4) (layers "F.Cu" "B.Cu") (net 8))
 (via (at 102.905 100.84) (size 0.8) (drill 0.4) (layers "F.Cu" "B.Cu") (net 8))
 (segment (start 100.282309 107.511389) (end 100.282309 103.462691) (width 0.25) (layer "B.Cu") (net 8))
 (segment (start 100.282309 103.462691) (end 102.905 100.84) (width 0.25) (layer "B.Cu") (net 8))
 (segment (start 101.07 101.73) (end 101.07 101.1425) (width 0.25) (layer "F.Cu") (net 7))
 (segment (start 102.905 99.310038) (end 102.905 99.0075) (width 0.25) (layer "F.Cu") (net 7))
 (segment (start 102.905 99.3075) (end 102.905 99.0075) (width 0.25) (layer "F.Cu") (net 7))
 (segment (start 99.28 107.508708) (end 99.282821 107.505887) (width 0.25) (layer "F.Cu") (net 7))
 (segment (start 101.07 101.1425) (end 102.905 99.3075) (width 0.25) (layer "F.Cu") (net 7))
 (segment (start 99.28 108.4925) (end 99.28 107.508708) (width 0.25) (layer "F.Cu") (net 7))
 (via (at 99.282821 107.505887) (size 0.8) (drill 0.4) (layers "F.Cu" "B.Cu") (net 7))
 (via (at 102.905 99.0075) (size 0.8) (drill 0.4) (layers "F.Cu" "B.Cu") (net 7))
 (segment (start 99.2975 102.615) (end 102.905 99.0075) (width 0.25) (layer "B.Cu") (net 7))
 (segment (start 99.282821 107.505887) (end 99.2975 107.491208) (width 0.25) (layer "B.Cu") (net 7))
 (segment (start 99.2975 107.491208) (end 99.2975 102.615) (width 0.25) (layer "B.Cu") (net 7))
 (segment (start 96.4325 103.6425) (end 95.865317 103.6425) (width 0.25) (layer "F.Cu") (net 9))
 (segment (start 95.66 103.847817) (end 95.66 105.665) (width 0.25) (layer "F.Cu") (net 9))
 (segment (start 95.865317 103.6425) (end 95.66 103.847817) (width 0.25) (layer "F.Cu") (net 9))
 (segment (start 95.66 105.665) (end 94.86 106.465) (width 0.25) (layer "F.Cu") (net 9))
 (segment (start 99.07 105.9775) (end 99.07 105.055) (width 0.25) (layer "F.Cu") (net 10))
 (segment (start 99.525 106.4325) (end 99.07 105.9775) (width 0.25) (layer "F.Cu") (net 10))
 (segment (start 99.07 99.62) (end 100.165 99.62) (width 0.25) (layer "F.Cu") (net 3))
 (segment (start 100.165 99.62) (end 100.61 100.065) (width 0.25) (layer "F.Cu") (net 3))
 (segment (start 98.07 100.62) (end 98.07 101.73) (width 0.25) (layer "F.Cu") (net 3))
 (segment (start 98.07 100.62) (end 99.07 99.62) (width 0.25) (layer "F.Cu") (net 3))
 (segment (start 96.57 99.62) (end 97.57 100.62) (width 0.25) (layer "F.Cu") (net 4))
 (segment (start 95.47 99.62) (end 95.03 100.06) (width 0.25) (layer "F.Cu") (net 4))
 (segment (start 96.57 99.62) (end 95.47 99.62) (width 0.25) (layer "F.Cu") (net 4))
 (segment (start 97.57 100.62) (end 97.57 101.73) (width 0.25) (layer "F.Cu") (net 4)))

